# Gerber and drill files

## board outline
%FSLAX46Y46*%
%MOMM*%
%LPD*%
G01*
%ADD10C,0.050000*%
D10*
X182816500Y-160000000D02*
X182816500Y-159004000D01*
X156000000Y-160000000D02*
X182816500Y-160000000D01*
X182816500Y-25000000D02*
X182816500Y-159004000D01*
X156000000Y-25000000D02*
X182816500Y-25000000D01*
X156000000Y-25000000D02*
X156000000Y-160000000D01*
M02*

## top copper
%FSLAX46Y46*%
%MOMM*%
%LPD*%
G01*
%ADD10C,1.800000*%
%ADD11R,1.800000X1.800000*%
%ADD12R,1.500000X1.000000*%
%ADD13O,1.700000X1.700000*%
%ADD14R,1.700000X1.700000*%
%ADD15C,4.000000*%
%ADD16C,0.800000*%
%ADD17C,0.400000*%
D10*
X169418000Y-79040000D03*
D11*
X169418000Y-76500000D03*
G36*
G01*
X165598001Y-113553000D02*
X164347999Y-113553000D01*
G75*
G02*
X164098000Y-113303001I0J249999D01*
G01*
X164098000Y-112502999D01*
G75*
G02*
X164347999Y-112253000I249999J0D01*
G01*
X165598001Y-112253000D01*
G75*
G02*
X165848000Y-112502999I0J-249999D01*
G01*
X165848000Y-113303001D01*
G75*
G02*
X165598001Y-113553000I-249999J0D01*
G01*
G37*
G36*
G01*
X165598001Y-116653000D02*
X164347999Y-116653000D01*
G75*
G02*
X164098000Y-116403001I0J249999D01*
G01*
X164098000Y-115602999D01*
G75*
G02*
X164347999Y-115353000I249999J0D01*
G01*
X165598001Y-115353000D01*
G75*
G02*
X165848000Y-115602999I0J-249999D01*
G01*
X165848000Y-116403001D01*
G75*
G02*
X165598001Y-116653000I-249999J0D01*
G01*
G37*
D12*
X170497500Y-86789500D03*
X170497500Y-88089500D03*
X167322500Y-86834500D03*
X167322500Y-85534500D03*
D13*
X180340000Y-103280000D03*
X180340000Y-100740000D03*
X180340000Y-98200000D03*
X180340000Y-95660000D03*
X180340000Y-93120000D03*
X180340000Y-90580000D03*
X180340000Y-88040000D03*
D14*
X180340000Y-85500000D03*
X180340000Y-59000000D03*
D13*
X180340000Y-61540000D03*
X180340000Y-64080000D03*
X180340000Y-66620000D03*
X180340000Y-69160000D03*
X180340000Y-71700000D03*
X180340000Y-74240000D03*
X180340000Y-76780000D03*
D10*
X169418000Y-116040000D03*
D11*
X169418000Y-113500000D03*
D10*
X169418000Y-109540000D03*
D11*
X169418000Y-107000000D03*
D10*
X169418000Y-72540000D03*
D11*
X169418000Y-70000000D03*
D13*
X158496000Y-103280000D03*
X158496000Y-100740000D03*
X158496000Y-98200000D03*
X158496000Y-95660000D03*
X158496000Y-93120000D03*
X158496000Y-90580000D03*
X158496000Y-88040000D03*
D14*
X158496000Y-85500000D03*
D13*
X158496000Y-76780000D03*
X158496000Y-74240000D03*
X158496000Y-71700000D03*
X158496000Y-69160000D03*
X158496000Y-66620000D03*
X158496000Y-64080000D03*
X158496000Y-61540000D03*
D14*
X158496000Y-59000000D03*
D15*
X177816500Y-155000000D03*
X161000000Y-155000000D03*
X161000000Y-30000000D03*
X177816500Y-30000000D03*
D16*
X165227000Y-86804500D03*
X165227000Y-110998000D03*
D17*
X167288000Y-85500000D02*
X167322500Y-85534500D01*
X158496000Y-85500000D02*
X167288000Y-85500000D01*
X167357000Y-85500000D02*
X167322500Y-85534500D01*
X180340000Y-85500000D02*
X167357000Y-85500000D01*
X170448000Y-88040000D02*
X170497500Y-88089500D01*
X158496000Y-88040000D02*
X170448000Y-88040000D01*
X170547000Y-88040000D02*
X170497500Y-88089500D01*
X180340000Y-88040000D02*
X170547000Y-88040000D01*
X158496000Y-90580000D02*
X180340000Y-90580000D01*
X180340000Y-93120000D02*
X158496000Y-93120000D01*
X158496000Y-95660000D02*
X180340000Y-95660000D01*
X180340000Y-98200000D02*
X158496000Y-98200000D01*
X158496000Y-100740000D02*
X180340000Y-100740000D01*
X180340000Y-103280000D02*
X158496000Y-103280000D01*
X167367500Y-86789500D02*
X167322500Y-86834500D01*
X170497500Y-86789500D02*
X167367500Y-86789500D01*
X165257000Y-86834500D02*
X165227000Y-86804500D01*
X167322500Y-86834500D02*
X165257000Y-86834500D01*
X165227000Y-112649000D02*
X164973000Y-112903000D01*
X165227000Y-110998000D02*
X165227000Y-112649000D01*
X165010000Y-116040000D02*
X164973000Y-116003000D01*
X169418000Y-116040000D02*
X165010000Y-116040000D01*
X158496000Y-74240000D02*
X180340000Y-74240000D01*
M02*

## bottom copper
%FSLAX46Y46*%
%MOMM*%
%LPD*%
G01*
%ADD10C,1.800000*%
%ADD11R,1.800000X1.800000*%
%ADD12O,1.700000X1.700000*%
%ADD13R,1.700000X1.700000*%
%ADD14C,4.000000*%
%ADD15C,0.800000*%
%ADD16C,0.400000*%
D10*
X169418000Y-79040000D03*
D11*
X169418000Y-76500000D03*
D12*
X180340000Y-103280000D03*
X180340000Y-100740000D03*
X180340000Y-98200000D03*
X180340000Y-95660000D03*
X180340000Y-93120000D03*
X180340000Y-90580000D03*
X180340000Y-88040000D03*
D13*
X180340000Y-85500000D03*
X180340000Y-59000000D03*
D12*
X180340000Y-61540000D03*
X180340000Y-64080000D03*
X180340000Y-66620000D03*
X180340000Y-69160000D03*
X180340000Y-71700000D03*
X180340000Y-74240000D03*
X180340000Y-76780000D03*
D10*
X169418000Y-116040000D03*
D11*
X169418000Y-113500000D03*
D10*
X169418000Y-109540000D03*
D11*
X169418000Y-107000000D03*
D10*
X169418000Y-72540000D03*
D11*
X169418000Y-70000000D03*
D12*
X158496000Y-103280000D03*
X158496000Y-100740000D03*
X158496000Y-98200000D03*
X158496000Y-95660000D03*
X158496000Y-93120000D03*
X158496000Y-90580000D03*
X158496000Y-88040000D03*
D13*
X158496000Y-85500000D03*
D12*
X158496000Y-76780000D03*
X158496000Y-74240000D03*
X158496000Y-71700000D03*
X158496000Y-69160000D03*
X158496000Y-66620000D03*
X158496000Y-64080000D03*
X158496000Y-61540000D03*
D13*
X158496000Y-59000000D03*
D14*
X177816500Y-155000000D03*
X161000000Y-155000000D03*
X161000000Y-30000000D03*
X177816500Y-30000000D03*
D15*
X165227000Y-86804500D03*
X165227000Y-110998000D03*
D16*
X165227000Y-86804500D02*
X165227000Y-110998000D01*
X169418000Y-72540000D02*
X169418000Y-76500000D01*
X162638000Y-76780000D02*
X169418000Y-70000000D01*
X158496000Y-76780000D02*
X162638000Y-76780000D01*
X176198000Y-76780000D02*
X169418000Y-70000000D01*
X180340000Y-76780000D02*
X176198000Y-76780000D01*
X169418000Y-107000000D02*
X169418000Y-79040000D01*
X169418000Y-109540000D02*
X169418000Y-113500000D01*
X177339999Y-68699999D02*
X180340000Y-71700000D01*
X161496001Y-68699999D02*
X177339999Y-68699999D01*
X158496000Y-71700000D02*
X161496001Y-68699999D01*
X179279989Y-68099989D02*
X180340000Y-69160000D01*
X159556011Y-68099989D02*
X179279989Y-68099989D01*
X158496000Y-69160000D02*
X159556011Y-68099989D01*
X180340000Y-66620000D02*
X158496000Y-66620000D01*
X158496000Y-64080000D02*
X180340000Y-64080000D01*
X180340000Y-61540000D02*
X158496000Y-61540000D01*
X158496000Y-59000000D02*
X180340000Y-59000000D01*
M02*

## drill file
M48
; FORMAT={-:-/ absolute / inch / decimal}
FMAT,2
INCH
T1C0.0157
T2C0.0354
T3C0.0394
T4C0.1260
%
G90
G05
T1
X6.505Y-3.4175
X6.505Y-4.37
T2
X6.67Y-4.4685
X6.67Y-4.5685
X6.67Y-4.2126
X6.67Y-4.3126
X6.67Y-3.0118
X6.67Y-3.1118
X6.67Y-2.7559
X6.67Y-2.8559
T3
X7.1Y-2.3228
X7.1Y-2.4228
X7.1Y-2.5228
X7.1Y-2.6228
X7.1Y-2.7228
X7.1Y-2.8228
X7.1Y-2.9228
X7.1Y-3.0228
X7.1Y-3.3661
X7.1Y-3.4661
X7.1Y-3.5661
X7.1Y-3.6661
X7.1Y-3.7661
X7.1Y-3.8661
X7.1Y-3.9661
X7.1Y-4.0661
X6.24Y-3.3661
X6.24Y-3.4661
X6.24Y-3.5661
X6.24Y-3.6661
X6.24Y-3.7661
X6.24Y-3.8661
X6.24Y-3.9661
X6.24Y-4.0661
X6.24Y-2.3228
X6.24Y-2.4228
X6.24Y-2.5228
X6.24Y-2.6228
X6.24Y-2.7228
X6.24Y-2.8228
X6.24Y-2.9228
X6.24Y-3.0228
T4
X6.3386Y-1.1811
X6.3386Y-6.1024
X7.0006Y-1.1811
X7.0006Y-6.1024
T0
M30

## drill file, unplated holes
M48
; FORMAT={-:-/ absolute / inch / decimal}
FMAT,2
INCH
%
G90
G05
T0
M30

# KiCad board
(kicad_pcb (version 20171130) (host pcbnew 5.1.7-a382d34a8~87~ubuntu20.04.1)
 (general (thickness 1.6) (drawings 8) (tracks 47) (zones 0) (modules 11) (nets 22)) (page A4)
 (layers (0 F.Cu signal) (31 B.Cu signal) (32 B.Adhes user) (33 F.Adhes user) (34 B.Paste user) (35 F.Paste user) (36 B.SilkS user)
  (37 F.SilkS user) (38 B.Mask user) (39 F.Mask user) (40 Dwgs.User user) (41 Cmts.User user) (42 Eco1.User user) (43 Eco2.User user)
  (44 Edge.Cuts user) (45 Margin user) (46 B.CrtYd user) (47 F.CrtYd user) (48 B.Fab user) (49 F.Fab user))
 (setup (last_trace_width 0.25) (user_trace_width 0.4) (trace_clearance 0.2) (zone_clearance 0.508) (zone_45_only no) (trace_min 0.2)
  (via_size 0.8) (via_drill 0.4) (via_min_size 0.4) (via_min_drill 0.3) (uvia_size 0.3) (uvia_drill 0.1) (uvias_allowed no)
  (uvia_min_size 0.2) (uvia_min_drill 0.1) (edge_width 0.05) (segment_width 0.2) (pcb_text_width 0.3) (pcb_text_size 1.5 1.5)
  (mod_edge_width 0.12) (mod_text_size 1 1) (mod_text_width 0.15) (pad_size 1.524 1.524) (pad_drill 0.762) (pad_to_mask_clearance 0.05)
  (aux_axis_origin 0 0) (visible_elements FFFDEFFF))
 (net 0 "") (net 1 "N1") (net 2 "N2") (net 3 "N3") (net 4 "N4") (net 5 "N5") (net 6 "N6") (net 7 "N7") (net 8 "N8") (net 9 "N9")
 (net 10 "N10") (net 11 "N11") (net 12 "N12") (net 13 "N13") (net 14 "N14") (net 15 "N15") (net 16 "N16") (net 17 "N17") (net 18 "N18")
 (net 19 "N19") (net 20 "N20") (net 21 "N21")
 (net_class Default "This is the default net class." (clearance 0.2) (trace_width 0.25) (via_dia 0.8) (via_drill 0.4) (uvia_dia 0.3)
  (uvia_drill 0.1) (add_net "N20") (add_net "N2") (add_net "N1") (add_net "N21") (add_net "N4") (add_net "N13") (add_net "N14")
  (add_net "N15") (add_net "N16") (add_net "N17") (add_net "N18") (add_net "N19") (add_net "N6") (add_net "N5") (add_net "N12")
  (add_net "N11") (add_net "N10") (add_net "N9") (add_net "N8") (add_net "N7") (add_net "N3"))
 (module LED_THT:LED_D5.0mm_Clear (layer F.Cu) (at 169.418 76.5 270)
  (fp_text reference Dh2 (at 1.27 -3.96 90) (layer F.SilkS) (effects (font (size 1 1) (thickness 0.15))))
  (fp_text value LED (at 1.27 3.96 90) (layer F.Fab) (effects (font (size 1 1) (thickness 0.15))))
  (pad 2 thru_hole circle (at 2.54 0 270) (size 1.8 1.8) (drill 0.9) (layers *.Cu *.Mask) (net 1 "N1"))
  (pad 1 thru_hole rect (at 0 0 270) (size 1.8 1.8) (drill 0.9) (layers *.Cu *.Mask) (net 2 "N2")))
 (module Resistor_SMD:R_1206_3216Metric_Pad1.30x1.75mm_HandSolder (layer F.Cu) (at 164.973 114.453 90)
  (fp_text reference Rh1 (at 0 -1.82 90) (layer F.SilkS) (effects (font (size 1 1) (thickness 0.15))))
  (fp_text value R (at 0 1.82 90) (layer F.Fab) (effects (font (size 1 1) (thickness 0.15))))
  (pad 2 smd roundrect (at 1.55 0 90) (size 1.3 1.75) (layers F.Cu F.Paste F.Mask) (roundrect_rratio 0.1923076923076923) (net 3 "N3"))
  (pad 1 smd roundrect (at -1.55 0 90) (size 1.3 1.75) (layers F.Cu F.Paste F.Mask) (roundrect_rratio 0.1923076923076923) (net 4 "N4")))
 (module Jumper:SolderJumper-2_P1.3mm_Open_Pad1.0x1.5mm (layer F.Cu) (at 170.4975 87.4395 270)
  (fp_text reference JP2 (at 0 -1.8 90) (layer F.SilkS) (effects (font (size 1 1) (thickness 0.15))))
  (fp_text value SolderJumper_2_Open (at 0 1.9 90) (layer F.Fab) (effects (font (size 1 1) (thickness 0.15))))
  (pad 1 smd rect (at -0.65 0 270) (size 1 1.5) (layers F.Cu F.Mask) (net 3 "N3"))
  (pad 2 smd rect (at 0.65 0 270) (size 1 1.5) (layers F.Cu F.Mask) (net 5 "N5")))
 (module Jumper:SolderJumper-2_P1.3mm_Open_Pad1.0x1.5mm (layer F.Cu) (at 167.3225 86.1845 90)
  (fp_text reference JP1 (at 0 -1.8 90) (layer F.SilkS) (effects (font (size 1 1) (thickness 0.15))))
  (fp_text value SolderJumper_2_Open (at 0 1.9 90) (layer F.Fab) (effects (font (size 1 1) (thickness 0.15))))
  (pad 1 smd rect (at -0.65 0 90) (size 1 1.5) (layers F.Cu F.Mask) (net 3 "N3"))
  (pad 2 smd rect (at 0.65 0 90) (size 1 1.5) (layers F.Cu F.Mask) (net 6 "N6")))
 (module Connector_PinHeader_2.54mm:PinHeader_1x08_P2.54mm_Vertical (layer F.Cu) (at 180.34 85.5)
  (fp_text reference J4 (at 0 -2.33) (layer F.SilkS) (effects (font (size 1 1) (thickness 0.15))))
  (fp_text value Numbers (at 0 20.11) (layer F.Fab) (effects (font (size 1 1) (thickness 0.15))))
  (pad 8 thru_hole oval (at 0 17.78) (size 1.7 1.7) (drill 1) (layers *.Cu *.Mask) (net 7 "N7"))
  (pad 7 thru_hole oval (at 0 15.24) (size 1.7 1.7) (drill 1) (layers *.Cu *.Mask) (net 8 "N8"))
  (pad 6 thru_hole oval (at 0 12.7) (size 1.7 1.7) (drill 1) (layers *.Cu *.Mask) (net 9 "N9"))
  (pad 5 thru_hole oval (at 0 10.16) (size 1.7 1.7) (drill 1) (layers *.Cu *.Mask) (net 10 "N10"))
  (pad 4 thru_hole oval (at 0 7.62) (size 1.7 1.7) (drill 1) (layers *.Cu *.Mask) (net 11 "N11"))
  (pad 3 thru_hole oval (at 0 5.08) (size 1.7 1.7) (drill 1) (layers *.Cu *.Mask) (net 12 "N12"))
  (pad 2 thru_hole oval (at 0 2.54) (size 1.7 1.7) (drill 1) (layers *.Cu *.Mask) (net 5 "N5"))
  (pad 1 thru_hole rect (at 0 0) (size 1.7 1.7) (drill 1) (layers *.Cu *.Mask) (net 6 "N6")))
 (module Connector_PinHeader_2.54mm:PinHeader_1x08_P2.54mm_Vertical (layer F.Cu) (at 180.34 59)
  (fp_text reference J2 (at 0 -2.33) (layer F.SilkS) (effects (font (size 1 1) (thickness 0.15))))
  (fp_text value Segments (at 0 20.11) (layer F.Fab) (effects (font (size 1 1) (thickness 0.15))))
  (pad 1 thru_hole rect (at 0 0) (size 1.7 1.7) (drill 1) (layers *.Cu *.Mask) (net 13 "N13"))
  (pad 2 thru_hole oval (at 0 2.54) (size 1.7 1.7) (drill 1) (layers *.Cu *.Mask) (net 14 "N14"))
  (pad 3 thru_hole oval (at 0 5.08) (size 1.7 1.7) (drill 1) (layers *.Cu *.Mask) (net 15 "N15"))
  (pad 4 thru_hole oval (at 0 7.62) (size 1.7 1.7) (drill 1) (layers *.Cu *.Mask) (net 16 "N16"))
  (pad 5 thru_hole oval (at 0 10.16) (size 1.7 1.7) (drill 1) (layers *.Cu *.Mask) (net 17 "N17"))
  (pad 6 thru_hole oval (at 0 12.7) (size 1.7 1.7) (drill 1) (layers *.Cu *.Mask) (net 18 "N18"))
  (pad 7 thru_hole oval (at 0 15.24) (size 1.7 1.7) (drill 1) (layers *.Cu *.Mask) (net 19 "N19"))
  (pad 8 thru_hole oval (at 0 17.78) (size 1.7 1.7) (drill 1) (layers *.Cu *.Mask) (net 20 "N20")))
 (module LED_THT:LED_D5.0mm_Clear (layer F.Cu) (at 169.418 113.5 270)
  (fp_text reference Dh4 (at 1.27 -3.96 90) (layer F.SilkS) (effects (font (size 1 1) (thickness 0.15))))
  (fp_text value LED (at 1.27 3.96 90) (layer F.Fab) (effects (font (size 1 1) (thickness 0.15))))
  (pad 2 thru_hole circle (at 2.54 0 270) (size 1.8 1.8) (drill 0.9) (layers *.Cu *.Mask) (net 4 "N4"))
  (pad 1 thru_hole rect (at 0 0 270) (size 1.8 1.8) (drill 0.9) (layers *.Cu *.Mask) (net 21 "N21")))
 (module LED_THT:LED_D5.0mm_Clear (layer F.Cu) (at 169.418 107 270)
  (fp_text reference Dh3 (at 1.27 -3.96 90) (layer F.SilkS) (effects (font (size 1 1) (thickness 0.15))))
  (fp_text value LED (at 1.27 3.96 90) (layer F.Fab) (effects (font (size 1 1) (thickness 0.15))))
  (pad 2 thru_hole circle (at 2.54 0 270) (size 1.8 1.8) (drill 0.9) (layers *.Cu *.Mask) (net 21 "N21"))
  (pad 1 thru_hole rect (at 0 0 270) (size 1.8 1.8) (drill 0.9) (layers *.Cu *.Mask) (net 1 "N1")))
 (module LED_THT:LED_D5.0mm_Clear (layer F.Cu) (at 169.418 70 270)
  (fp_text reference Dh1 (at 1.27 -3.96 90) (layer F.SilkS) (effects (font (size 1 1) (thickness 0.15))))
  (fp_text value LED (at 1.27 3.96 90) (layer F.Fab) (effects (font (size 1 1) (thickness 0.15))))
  (pad 2 thru_hole circle (at 2.54 0 270) (size 1.8 1.8) (drill 0.9) (layers *.Cu *.Mask) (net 2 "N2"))
  (pad 1 thru_hole rect (at 0 0 270) (size 1.8 1.8) (drill 0.9) (layers *.Cu *.Mask) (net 20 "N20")))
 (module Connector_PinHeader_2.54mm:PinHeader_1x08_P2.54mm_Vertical (layer F.Cu) (at 158.496 85.5)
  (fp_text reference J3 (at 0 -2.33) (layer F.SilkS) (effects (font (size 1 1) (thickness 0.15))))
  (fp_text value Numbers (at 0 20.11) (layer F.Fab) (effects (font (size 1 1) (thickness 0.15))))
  (pad 8 thru_hole oval (at 0 17.78) (size 1.7 1.7) (drill 1) (layers *.Cu *.Mask) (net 7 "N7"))
  (pad 7 thru_hole oval (at 0 15.24) (size 1.7 1.7) (drill 1) (layers *.Cu *.Mask) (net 8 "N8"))
  (pad 6 thru_hole oval (at 0 12.7) (size 1.7 1.7) (drill 1) (layers *.Cu *.Mask) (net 9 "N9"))
  (pad 5 thru_hole oval (at 0 10.16) (size 1.7 1.7) (drill 1) (layers *.Cu *.Mask) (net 10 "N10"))
  (pad 4 thru_hole oval (at 0 7.62) (size 1.7 1.7) (drill 1) (layers *.Cu *.Mask) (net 11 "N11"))
  (pad 3 thru_hole oval (at 0 5.08) (size 1.7 1.7) (drill 1) (layers *.Cu *.Mask) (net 12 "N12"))
  (pad 2 thru_hole oval (at 0 2.54) (size 1.7 1.7) (drill 1) (layers *.Cu *.Mask) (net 5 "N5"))
  (pad 1 thru_hole rect (at 0 0) (size 1.7 1.7) (drill 1) (layers *.Cu *.Mask) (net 6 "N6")))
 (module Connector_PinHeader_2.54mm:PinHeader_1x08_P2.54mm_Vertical (layer F.Cu) (at 158.496 59)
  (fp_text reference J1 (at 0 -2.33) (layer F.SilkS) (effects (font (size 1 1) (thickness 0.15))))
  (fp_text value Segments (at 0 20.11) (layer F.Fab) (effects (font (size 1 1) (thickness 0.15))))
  (pad 8 thru_hole oval (at 0 17.78) (size 1.7 1.7) (drill 1) (layers *.Cu *.Mask) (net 20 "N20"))
  (pad 7 thru_hole oval (at 0 15.24) (size 1.7 1.7) (drill 1) (layers *.Cu *.Mask) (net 19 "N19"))
  (pad 6 thru_hole oval (at 0 12.7) (size 1.7 1.7) (drill 1) (layers *.Cu *.Mask) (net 18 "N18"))
  (pad 5 thru_hole oval (at 0 10.16) (size 1.7 1.7) (drill 1) (layers *.Cu *.Mask) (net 17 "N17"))
  (pad 4 thru_hole oval (at 0 7.62) (size 1.7 1.7) (drill 1) (layers *.Cu *.Mask) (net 16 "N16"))
  (pad 3 thru_hole oval (at 0 5.08) (size 1.7 1.7) (drill 1) (layers *.Cu *.Mask) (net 15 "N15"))
  (pad 2 thru_hole oval (at 0 2.54) (size 1.7 1.7) (drill 1) (layers *.Cu *.Mask) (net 14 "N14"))
  (pad 1 thru_hole rect (at 0 0) (size 1.7 1.7) (drill 1) (layers *.Cu *.Mask) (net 13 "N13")))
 (gr_line (start 182.8165 160) (end 182.8165 159.004) (layer Edge.Cuts) (width 0.05))
 (gr_line (start 156 160) (end 182.8165 160) (layer Edge.Cuts) (width 0.05))
 (gr_line (start 182.8165 25) (end 182.8165 159.004) (layer Edge.Cuts) (width 0.05))
 (gr_line (start 156 25) (end 182.8165 25) (layer Edge.Cuts) (width 0.05))
 (gr_line (start 156 25) (end 156 160) (layer Edge.Cuts) (width 0.05))
 (via (at 177.8165 155) (size 4) (drill 3.2) (layers F.Cu B.Cu) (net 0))
 (via (at 161 155) (size 4) (drill 3.2) (layers F.Cu B.Cu) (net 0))
 (via (at 161 30) (size 4) (drill 3.2) (layers F.Cu B.Cu) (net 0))
 (via (at 177.8165 30) (size 4) (drill 3.2) (layers F.Cu B.Cu) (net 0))
 (segment (start 167.288 85.5) (end 167.3225 85.5345) (width 0.4) (layer F.Cu) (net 6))
 (segment (start 158.496 85.5) (end 167.288 85.5) (width 0.4) (layer F.Cu) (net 6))
 (segment (start 167.357 85.5) (end 167.3225 85.5345) (width 0.4) (layer F.Cu) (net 6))
 (segment (start 180.34 85.5) (end 167.357 85.5) (width 0.4) (layer F.Cu) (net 6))
 (segment (start 170.448 88.04) (end 170.4975 88.0895) (width 0.4) (layer F.Cu) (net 5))
 (segment (start 158.496 88.04) (end 170.448 88.04) (width 0.4) (layer F.Cu) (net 5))
 (segment (start 170.547 88.04) (end 170.4975 88.0895) (width 0.4) (layer F.Cu) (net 5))
 (segment (start 180.34 88.04) (end 170.547 88.04) (width 0.4) (layer F.Cu) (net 5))
 (segment (start 158.496 90.58) (end 180.34 90.58) (width 0.4) (layer F.Cu) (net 12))
 (segment (start 180.34 93.12) (end 158.496 93.12) (width 0.4) (layer F.Cu) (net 11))
 (segment (start 158.496 95.66) (end 180.34 95.66) (width 0.4) (layer F.Cu) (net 10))
 (segment (start 180.34 98.2) (end 158.496 98.2) (width 0.4) (layer F.Cu) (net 9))
 (segment (start 158.496 100.74) (end 180.34 100.74) (width 0.4) (layer F.Cu) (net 8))
 (segment (start 180.34 103.28) (end 158.496 103.28) (width 0.4) (layer F.Cu) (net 7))
 (segment (start 167.3675 86.7895) (end 167.3225 86.8345) (width 0.4) (layer F.Cu) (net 3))
 (segment (start 170.4975 86.7895) (end 167.3675 86.7895) (width 0.4) (layer F.Cu) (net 3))
 (via (at 165.227 86.8045) (size 0.8) (drill 0.4) (layers F.Cu B.Cu) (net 3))
 (segment (start 165.257 86.8345) (end 165.227 86.8045) (width 0.4) (layer F.Cu) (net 3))
 (segment (start 167.3225 86.8345) (end 165.257 86.8345) (width 0.4) (layer F.Cu) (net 3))
 (via (at 165.227 110.998) (size 0.8) (drill 0.4) (layers F.Cu B.Cu) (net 3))
 (segment (start 165.227 86.8045) (end 165.227 110.998) (width 0.4) (layer B.Cu) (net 3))
 (segment (start 165.227 112.649) (end 164.973 112.903) (width 0.4) (layer F.Cu) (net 3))
 (segment (start 165.227 110.998) (end 165.227 112.649) (width 0.4) (layer F.Cu) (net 3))
 (segment (start 169.418 72.54) (end 169.418 76.5) (width 0.4) (layer B.Cu) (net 2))
 (segment (start 162.638 76.78) (end 169.418 70) (width 0.4) (layer B.Cu) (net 20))
 (segment (start 158.496 76.78) (end 162.638 76.78) (width 0.4) (layer B.Cu) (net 20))
 (segment (start 176.198 76.78) (end 169.418 70) (width 0.4) (layer B.Cu) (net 20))
 (segment (start 180.34 76.78) (end 176.198 76.78) (width 0.4) (layer B.Cu) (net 20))
 (segment (start 169.418 107) (end 169.418 79.04) (width 0.4) (layer B.Cu) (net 1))
 (segment (start 169.418 109.54) (end 169.418 113.5) (width 0.4) (layer B.Cu) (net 21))
 (segment (start 165.01 116.04) (end 164.973 116.003) (width 0.4) (layer F.Cu) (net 4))
 (segment (start 169.418 116.04) (end 165.01 116.04) (width 0.4) (layer F.Cu) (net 4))
 (segment (start 158.496 74.24) (end 180.34 74.24) (width 0.4) (layer F.Cu) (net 19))
 (segment (start 177.339999 68.699999) (end 180.34 71.7) (width 0.4) (layer B.Cu) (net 18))
 (segment (start 161.496001 68.699999) (end 177.339999 68.699999) (width 0.4) (layer B.Cu) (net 18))
 (segment (start 158.496 71.7) (end 161.496001 68.699999) (width 0.4) (layer B.Cu) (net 18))
 (segment (start 179.279989 68.099989) (end 180.34 69.16) (width 0.4) (layer B.Cu) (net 17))
 (segment (start 159.556011 68.099989) (end 179.279989 68.099989) (width 0.4) (layer B.Cu) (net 17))
 (segment (start 158.496 69.16) (end 159.556011 68.099989) (width 0.4) (layer B.Cu) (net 17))
 (segment (start 180.34 66.62) (end 158.496 66.62) (width 0.4) (layer B.Cu) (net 16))
 (segment (start 158.496 64.08) (end 180.34 64.08) (width 0.4) (layer B.Cu) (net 15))
 (segment (start 180.34 61.54) (end 158.496 61.54) (width 0.4) (layer B.Cu) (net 14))
 (segment (start 158.496 59) (end 180.34 59) (width 0.4) (layer B.Cu) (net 13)))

